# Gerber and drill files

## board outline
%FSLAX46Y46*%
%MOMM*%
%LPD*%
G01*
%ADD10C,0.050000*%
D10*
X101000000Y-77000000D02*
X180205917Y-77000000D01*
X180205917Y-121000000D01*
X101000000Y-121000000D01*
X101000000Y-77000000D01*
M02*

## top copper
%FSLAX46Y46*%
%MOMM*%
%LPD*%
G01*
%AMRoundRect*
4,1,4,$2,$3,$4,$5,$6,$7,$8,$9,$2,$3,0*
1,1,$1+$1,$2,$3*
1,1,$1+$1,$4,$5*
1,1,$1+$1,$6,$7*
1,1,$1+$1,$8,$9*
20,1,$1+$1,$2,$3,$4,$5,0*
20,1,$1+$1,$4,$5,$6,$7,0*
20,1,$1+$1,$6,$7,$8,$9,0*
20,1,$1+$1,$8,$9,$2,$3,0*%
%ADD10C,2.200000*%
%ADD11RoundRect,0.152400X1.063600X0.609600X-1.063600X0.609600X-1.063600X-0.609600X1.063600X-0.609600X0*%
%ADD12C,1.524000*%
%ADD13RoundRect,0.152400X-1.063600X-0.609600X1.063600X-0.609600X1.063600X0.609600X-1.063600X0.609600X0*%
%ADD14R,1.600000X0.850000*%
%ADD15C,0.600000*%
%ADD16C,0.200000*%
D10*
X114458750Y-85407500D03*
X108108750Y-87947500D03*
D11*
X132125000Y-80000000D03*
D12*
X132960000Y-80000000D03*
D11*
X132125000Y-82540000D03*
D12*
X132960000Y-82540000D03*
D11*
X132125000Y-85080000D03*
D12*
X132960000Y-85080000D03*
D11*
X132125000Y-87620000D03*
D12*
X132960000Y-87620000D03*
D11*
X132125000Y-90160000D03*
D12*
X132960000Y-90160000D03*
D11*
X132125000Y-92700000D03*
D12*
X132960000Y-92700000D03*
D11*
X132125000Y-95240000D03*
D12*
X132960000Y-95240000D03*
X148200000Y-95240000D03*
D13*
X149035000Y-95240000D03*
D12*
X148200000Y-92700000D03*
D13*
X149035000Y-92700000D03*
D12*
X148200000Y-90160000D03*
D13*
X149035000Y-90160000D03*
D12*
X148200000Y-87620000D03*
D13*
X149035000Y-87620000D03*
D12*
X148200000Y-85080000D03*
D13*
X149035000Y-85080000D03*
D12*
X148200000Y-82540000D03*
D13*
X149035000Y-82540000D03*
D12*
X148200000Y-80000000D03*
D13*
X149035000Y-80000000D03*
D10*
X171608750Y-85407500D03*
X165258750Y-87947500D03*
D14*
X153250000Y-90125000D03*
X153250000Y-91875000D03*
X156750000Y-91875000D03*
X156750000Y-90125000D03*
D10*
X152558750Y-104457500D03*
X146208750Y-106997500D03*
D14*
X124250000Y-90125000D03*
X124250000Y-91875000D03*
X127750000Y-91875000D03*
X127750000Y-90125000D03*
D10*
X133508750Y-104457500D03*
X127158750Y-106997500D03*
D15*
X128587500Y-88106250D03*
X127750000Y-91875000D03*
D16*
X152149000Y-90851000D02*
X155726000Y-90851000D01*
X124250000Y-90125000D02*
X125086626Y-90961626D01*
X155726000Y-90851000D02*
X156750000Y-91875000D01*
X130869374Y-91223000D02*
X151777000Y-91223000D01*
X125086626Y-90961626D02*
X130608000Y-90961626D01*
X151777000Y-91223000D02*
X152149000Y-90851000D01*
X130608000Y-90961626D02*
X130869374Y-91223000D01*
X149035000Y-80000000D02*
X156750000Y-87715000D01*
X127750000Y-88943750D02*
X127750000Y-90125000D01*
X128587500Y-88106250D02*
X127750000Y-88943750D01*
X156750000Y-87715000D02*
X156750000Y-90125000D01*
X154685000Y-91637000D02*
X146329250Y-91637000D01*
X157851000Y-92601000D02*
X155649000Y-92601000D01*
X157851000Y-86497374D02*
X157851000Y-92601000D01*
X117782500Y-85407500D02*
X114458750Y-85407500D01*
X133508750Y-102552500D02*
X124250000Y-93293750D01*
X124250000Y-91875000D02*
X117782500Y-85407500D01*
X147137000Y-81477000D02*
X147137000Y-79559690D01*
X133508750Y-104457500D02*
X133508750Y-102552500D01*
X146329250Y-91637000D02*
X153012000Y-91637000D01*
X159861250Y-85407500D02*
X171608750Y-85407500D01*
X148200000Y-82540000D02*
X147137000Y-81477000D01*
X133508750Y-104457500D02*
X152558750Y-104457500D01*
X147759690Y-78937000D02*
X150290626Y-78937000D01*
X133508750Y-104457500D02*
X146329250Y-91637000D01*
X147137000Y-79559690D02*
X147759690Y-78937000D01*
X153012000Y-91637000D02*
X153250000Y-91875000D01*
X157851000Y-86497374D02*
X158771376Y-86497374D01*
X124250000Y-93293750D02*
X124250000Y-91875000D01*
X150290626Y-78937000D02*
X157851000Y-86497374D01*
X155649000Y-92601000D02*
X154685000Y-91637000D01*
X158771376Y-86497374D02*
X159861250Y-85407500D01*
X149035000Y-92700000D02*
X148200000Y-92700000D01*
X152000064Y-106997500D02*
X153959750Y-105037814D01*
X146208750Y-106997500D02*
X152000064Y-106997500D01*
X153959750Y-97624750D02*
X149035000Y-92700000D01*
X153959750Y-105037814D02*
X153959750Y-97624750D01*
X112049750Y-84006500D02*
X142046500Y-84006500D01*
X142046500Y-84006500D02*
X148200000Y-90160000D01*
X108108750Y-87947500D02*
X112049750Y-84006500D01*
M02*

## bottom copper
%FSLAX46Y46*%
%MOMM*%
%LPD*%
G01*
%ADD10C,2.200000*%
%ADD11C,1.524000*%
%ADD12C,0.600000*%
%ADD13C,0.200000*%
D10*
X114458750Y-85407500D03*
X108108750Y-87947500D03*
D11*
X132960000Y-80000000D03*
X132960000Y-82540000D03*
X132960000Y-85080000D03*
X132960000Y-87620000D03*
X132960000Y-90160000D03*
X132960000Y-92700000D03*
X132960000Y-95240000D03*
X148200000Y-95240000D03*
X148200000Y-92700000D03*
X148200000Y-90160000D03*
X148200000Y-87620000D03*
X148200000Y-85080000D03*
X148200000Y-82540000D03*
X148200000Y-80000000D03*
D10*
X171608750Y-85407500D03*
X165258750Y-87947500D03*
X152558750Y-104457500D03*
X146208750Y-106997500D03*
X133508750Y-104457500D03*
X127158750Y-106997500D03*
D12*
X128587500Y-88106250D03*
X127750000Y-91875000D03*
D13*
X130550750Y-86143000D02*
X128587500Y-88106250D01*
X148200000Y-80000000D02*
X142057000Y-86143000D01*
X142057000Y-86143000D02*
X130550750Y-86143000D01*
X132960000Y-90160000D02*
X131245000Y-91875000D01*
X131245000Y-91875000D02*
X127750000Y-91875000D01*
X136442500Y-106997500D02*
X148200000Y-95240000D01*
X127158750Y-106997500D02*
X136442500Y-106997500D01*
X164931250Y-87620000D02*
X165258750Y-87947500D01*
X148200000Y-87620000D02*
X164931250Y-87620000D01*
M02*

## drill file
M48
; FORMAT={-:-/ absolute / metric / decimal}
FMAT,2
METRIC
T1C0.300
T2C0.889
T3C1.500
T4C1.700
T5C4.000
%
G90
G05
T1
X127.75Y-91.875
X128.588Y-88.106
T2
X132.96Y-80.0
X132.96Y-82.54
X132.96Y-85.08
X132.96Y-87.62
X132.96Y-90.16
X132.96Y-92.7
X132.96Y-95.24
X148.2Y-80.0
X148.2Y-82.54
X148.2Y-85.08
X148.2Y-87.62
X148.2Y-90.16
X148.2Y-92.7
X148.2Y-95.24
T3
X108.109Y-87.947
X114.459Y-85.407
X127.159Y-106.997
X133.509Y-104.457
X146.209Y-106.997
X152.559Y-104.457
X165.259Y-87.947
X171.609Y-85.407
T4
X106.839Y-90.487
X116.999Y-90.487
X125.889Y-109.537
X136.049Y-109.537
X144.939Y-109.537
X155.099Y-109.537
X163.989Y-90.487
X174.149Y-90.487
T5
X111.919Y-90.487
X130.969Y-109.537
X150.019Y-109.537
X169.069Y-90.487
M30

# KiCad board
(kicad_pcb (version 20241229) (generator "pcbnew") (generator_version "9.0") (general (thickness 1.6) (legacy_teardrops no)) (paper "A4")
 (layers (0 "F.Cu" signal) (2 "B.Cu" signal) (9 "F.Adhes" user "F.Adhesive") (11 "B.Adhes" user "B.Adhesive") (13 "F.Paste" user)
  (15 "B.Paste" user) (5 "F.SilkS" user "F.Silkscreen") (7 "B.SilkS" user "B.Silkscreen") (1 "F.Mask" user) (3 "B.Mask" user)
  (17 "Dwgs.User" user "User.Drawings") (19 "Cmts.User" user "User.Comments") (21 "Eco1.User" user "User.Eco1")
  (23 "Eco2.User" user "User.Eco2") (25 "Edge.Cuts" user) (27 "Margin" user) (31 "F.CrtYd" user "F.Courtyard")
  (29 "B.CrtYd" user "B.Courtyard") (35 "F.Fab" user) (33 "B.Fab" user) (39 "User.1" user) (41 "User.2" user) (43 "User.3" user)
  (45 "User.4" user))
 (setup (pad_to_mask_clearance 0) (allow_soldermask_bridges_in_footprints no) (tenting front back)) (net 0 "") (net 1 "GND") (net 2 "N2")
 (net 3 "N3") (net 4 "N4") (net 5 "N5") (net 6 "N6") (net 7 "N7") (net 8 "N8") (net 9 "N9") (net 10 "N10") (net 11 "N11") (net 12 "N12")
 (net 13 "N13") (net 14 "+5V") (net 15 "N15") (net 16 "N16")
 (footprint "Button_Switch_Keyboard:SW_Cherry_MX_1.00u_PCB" (layer "F.Cu") (at 114.45875 85.4075)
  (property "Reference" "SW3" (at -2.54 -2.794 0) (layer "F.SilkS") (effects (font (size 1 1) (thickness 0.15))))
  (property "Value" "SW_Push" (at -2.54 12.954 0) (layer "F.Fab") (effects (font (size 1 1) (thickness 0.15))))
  (pad "" np_thru_hole circle (at -7.62 5.08) (size 1.7 1.7) (drill 1.7) (layers "*.Cu" "*.Mask"))
  (pad "" np_thru_hole circle (at -2.54 5.08) (size 4 4) (drill 4) (layers "*.Cu" "*.Mask"))
  (pad "" np_thru_hole circle (at 2.54 5.08) (size 1.7 1.7) (drill 1.7) (layers "*.Cu" "*.Mask"))
  (pad "1" thru_hole circle (at 0 0) (size 2.2 2.2) (drill 1.5) (layers "*.Cu" "*.Mask") (remove_unused_layers no) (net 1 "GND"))
  (pad "2" thru_hole circle (at -6.35 2.54) (size 2.2 2.2) (drill 1.5) (layers "*.Cu" "*.Mask") (remove_unused_layers no) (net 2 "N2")))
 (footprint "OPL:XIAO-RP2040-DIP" (layer "F.Cu") (at 140.58 87.62)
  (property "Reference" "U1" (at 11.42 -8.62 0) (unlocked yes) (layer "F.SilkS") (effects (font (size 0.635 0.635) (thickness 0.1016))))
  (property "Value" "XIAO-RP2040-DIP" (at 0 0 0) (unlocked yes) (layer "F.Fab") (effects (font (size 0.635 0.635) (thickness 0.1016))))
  (pad "1" smd roundrect (at -8.455 -7.62 180) (size 2.432 1.524) (layers "F.Cu" "F.Mask") (roundrect_rratio 0.1) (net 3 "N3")
   (thermal_bridge_angle 45))
  (pad "1" thru_hole circle (at -7.62 -7.62 180) (size 1.524 1.524) (drill 0.889) (layers "*.Cu" "*.Mask") (remove_unused_layers no)
   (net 3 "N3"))
  (pad "2" smd roundrect (at -8.455 -5.08 180) (size 2.432 1.524) (layers "F.Cu" "F.Mask") (roundrect_rratio 0.1) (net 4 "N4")
   (thermal_bridge_angle 45))
  (pad "2" thru_hole circle (at -7.62 -5.08 180) (size 1.524 1.524) (drill 0.889) (layers "*.Cu" "*.Mask") (remove_unused_layers no)
   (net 4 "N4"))
  (pad "3" smd roundrect (at -8.455 -2.54 180) (size 2.432 1.524) (layers "F.Cu" "F.Mask") (roundrect_rratio 0.1) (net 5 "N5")
   (thermal_bridge_angle 45))
  (pad "3" thru_hole circle (at -7.62 -2.54 180) (size 1.524 1.524) (drill 0.889) (layers "*.Cu" "*.Mask") (remove_unused_layers no)
   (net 5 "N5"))
  (pad "4" smd roundrect (at -8.455 0 180) (size 2.432 1.524) (layers "F.Cu" "F.Mask") (roundrect_rratio 0.1) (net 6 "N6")
   (thermal_bridge_angle 45))
  (pad "4" thru_hole circle (at -7.62 0 180) (size 1.524 1.524) (drill 0.889) (layers "*.Cu" "*.Mask") (remove_unused_layers no)
   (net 6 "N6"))
  (pad "5" smd roundrect (at -8.455 2.54 180) (size 2.432 1.524) (layers "F.Cu" "F.Mask") (roundrect_rratio 0.1) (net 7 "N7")
   (thermal_bridge_angle 45))
  (pad "5" thru_hole circle (at -7.62 2.54 180) (size 1.524 1.524) (drill 0.889) (layers "*.Cu" "*.Mask") (remove_unused_layers no)
   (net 7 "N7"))
  (pad "6" smd roundrect (at -8.455 5.08 180) (size 2.432 1.524) (layers "F.Cu" "F.Mask") (roundrect_rratio 0.1) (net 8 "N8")
   (thermal_bridge_angle 45))
  (pad "6" thru_hole circle (at -7.62 5.08 180) (size 1.524 1.524) (drill 0.889) (layers "*.Cu" "*.Mask") (remove_unused_layers no)
   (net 8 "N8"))
  (pad "7" smd roundrect (at -8.455 7.62 180) (size 2.432 1.524) (layers "F.Cu" "F.Mask") (roundrect_rratio 0.1) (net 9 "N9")
   (thermal_bridge_angle 45))
  (pad "7" thru_hole circle (at -7.62 7.62 180) (size 1.524 1.524) (drill 0.889) (layers "*.Cu" "*.Mask") (remove_unused_layers no)
   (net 9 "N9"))
  (pad "8" thru_hole circle (at 7.62 7.62) (size 1.524 1.524) (drill 0.889) (layers "*.Cu" "*.Mask") (remove_unused_layers no)
   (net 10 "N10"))
  (pad "8" smd roundrect (at 8.455 7.62) (size 2.432 1.524) (layers "F.Cu" "F.Mask") (roundrect_rratio 0.1) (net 10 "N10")
   (thermal_bridge_angle 45))
  (pad "9" thru_hole circle (at 7.62 5.08) (size 1.524 1.524) (drill 0.889) (layers "*.Cu" "*.Mask") (remove_unused_layers no)
   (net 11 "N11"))
  (pad "9" smd roundrect (at 8.455 5.08) (size 2.432 1.524) (layers "F.Cu" "F.Mask") (roundrect_rratio 0.1) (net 11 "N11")
   (thermal_bridge_angle 45))
  (pad "10" thru_hole circle (at 7.62 2.54) (size 1.524 1.524) (drill 0.889) (layers "*.Cu" "*.Mask") (remove_unused_layers no) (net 2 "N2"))
  (pad "10" smd roundrect (at 8.455 2.54) (size 2.432 1.524) (layers "F.Cu" "F.Mask") (roundrect_rratio 0.1) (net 2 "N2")
   (thermal_bridge_angle 45))
  (pad "11" thru_hole circle (at 7.62 0) (size 1.524 1.524) (drill 0.889) (layers "*.Cu" "*.Mask") (remove_unused_layers no) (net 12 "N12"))
  (pad "11" smd roundrect (at 8.455 0) (size 2.432 1.524) (layers "F.Cu" "F.Mask") (roundrect_rratio 0.1) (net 12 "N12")
   (thermal_bridge_angle 45))
  (pad "12" thru_hole circle (at 7.62 -2.54) (size 1.524 1.524) (drill 0.889) (layers "*.Cu" "*.Mask") (remove_unused_layers no)
   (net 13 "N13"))
  (pad "12" smd roundrect (at 8.455 -2.54) (size 2.432 1.524) (layers "F.Cu" "F.Mask") (roundrect_rratio 0.1) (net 13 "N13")
   (thermal_bridge_angle 45))
  (pad "13" thru_hole circle (at 7.62 -5.08) (size 1.524 1.524) (drill 0.889) (layers "*.Cu" "*.Mask") (remove_unused_layers no)
   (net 1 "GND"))
  (pad "13" smd roundrect (at 8.455 -5.08) (size 2.432 1.524) (layers "F.Cu" "F.Mask") (roundrect_rratio 0.1) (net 1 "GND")
   (thermal_bridge_angle 45))
  (pad "14" thru_hole circle (at 7.62 -7.62) (size 1.524 1.524) (drill 0.889) (layers "*.Cu" "*.Mask") (remove_unused_layers no)
   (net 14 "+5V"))
  (pad "14" smd roundrect (at 8.455 -7.62) (size 2.432 1.524) (layers "F.Cu" "F.Mask") (roundrect_rratio 0.1) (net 14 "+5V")
   (thermal_bridge_angle 45)))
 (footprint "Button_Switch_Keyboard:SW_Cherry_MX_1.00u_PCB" (layer "F.Cu") (at 171.60875 85.4075)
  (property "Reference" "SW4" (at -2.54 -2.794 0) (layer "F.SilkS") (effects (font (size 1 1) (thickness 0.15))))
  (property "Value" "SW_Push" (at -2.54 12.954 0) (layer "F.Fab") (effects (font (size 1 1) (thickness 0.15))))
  (pad "" np_thru_hole circle (at -7.62 5.08) (size 1.7 1.7) (drill 1.7) (layers "*.Cu" "*.Mask"))
  (pad "" np_thru_hole circle (at -2.54 5.08) (size 4 4) (drill 4) (layers "*.Cu" "*.Mask"))
  (pad "" np_thru_hole circle (at 2.54 5.08) (size 1.7 1.7) (drill 1.7) (layers "*.Cu" "*.Mask"))
  (pad "1" thru_hole circle (at 0 0) (size 2.2 2.2) (drill 1.5) (layers "*.Cu" "*.Mask") (remove_unused_layers no) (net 1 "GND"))
  (pad "2" thru_hole circle (at -6.35 2.54) (size 2.2 2.2) (drill 1.5) (layers "*.Cu" "*.Mask") (remove_unused_layers no) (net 12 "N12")))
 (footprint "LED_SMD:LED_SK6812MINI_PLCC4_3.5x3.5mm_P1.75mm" (layer "F.Cu") (at 155 91)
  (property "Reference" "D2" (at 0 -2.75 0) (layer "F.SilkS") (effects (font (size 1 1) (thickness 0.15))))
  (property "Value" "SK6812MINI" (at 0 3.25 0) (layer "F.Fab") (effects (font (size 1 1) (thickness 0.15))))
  (pad "1" smd rect (at -1.75 -0.875) (size 1.6 0.85) (layers "F.Cu" "F.Mask" "F.Paste") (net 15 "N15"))
  (pad "2" smd rect (at -1.75 0.875) (size 1.6 0.85) (layers "F.Cu" "F.Mask" "F.Paste") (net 1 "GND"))
  (pad "3" smd rect (at 1.75 0.875) (size 1.6 0.85) (layers "F.Cu" "F.Mask" "F.Paste") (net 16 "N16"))
  (pad "4" smd rect (at 1.75 -0.875) (size 1.6 0.85) (layers "F.Cu" "F.Mask" "F.Paste") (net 14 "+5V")))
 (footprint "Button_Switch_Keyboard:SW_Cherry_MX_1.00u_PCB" (layer "F.Cu") (at 152.55875 104.4575)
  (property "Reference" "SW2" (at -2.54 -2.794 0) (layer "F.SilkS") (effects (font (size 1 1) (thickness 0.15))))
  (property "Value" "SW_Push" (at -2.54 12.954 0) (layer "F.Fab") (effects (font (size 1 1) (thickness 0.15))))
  (pad "" np_thru_hole circle (at -7.62 5.08) (size 1.7 1.7) (drill 1.7) (layers "*.Cu" "*.Mask"))
  (pad "" np_thru_hole circle (at -2.54 5.08) (size 4 4) (drill 4) (layers "*.Cu" "*.Mask"))
  (pad "" np_thru_hole circle (at 2.54 5.08) (size 1.7 1.7) (drill 1.7) (layers "*.Cu" "*.Mask"))
  (pad "1" thru_hole circle (at 0 0) (size 2.2 2.2) (drill 1.5) (layers "*.Cu" "*.Mask") (remove_unused_layers no) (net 1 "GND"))
  (pad "2" thru_hole circle (at -6.35 2.54) (size 2.2 2.2) (drill 1.5) (layers "*.Cu" "*.Mask") (remove_unused_layers no) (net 11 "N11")))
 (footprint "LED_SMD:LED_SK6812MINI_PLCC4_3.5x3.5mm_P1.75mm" (layer "F.Cu") (at 126 91)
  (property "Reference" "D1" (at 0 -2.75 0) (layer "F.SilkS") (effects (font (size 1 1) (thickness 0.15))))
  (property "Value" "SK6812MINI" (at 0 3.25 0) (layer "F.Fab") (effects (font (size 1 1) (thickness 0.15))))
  (pad "1" smd rect (at -1.75 -0.875) (size 1.6 0.85) (layers "F.Cu" "F.Mask" "F.Paste") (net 16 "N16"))
  (pad "2" smd rect (at -1.75 0.875) (size 1.6 0.85) (layers "F.Cu" "F.Mask" "F.Paste") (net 1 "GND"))
  (pad "3" smd rect (at 1.75 0.875) (size 1.6 0.85) (layers "F.Cu" "F.Mask" "F.Paste") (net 7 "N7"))
  (pad "4" smd rect (at 1.75 -0.875) (size 1.6 0.85) (layers "F.Cu" "F.Mask" "F.Paste") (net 14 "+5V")))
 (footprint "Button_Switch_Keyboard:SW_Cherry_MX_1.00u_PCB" (layer "F.Cu") (at 133.50875 104.4575)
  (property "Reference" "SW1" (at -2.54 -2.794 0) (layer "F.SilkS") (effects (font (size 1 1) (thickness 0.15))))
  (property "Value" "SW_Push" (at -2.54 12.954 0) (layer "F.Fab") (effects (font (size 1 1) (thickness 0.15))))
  (pad "" np_thru_hole circle (at -7.62 5.08) (size 1.7 1.7) (drill 1.7) (layers "*.Cu" "*.Mask"))
  (pad "" np_thru_hole circle (at -2.54 5.08) (size 4 4) (drill 4) (layers "*.Cu" "*.Mask"))
  (pad "" np_thru_hole circle (at 2.54 5.08) (size 1.7 1.7) (drill 1.7) (layers "*.Cu" "*.Mask"))
  (pad "1" thru_hole circle (at 0 0) (size 2.2 2.2) (drill 1.5) (layers "*.Cu" "*.Mask") (remove_unused_layers no) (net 1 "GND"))
  (pad "2" thru_hole circle (at -6.35 2.54) (size 2.2 2.2) (drill 1.5) (layers "*.Cu" "*.Mask") (remove_unused_layers no) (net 10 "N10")))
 (gr_rect (start 101 77) (end 180.205917 121) (stroke (width 0.05) (type default)) (fill no) (layer "Edge.Cuts"))
 (segment (start 152.149 90.851) (end 155.726 90.851) (width 0.2) (layer "F.Cu") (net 16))
 (segment (start 124.25 90.125) (end 125.086626 90.961626) (width 0.2) (layer "F.Cu") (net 16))
 (segment (start 155.726 90.851) (end 156.75 91.875) (width 0.2) (layer "F.Cu") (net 16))
 (segment (start 130.869374 91.223) (end 151.777 91.223) (width 0.2) (layer "F.Cu") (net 16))
 (segment (start 125.086626 90.961626) (end 130.608 90.961626) (width 0.2) (layer "F.Cu") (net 16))
 (segment (start 151.777 91.223) (end 152.149 90.851) (width 0.2) (layer "F.Cu") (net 16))
 (segment (start 130.608 90.961626) (end 130.869374 91.223) (width 0.2) (layer "F.Cu") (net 16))
 (segment (start 149.035 80) (end 156.75 87.715) (width 0.2) (layer "F.Cu") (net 14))
 (segment (start 127.75 88.94375) (end 127.75 90.125) (width 0.2) (layer "F.Cu") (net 14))
 (segment (start 128.5875 88.10625) (end 127.75 88.94375) (width 0.2) (layer "F.Cu") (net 14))
 (segment (start 156.75 87.715) (end 156.75 90.125) (width 0.2) (layer "F.Cu") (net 14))
 (via (at 128.5875 88.10625) (size 0.6) (drill 0.3) (layers "F.Cu" "B.Cu") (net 14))
 (segment (start 130.55075 86.143) (end 128.5875 88.10625) (width 0.2) (layer "B.Cu") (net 14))
 (segment (start 148.2 80) (end 142.057 86.143) (width 0.2) (layer "B.Cu") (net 14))
 (segment (start 142.057 86.143) (end 130.55075 86.143) (width 0.2) (layer "B.Cu") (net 14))
 (via (at 127.75 91.875) (size 0.6) (drill 0.3) (layers "F.Cu" "B.Cu") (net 7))
 (segment (start 132.96 90.16) (end 131.245 91.875) (width 0.2) (layer "B.Cu") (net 7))
 (segment (start 131.245 91.875) (end 127.75 91.875) (width 0.2) (layer "B.Cu") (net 7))
 (segment (start 154.685 91.637) (end 146.32925 91.637) (width 0.2) (layer "F.Cu") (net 1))
 (segment (start 157.851 92.601) (end 155.649 92.601) (width 0.2) (layer "F.Cu") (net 1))
 (segment (start 157.851 86.497374) (end 157.851 92.601) (width 0.2) (layer "F.Cu") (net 1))
 (segment (start 117.7825 85.4075) (end 114.45875 85.4075) (width 0.2) (layer "F.Cu") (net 1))
 (segment (start 133.50875 102.5525) (end 124.25 93.29375) (width 0.2) (layer "F.Cu") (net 1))
 (segment (start 124.25 91.875) (end 117.7825 85.4075) (width 0.2) (layer "F.Cu") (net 1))
 (segment (start 147.137 81.477) (end 147.137 79.55969) (width 0.2) (layer "F.Cu") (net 1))
 (segment (start 133.50875 104.4575) (end 133.50875 102.5525) (width 0.2) (layer "F.Cu") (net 1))
 (segment (start 146.32925 91.637) (end 153.012 91.637) (width 0.2) (layer "F.Cu") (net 1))
 (segment (start 159.86125 85.4075) (end 171.60875 85.4075) (width 0.2) (layer "F.Cu") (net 1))
 (segment (start 148.2 82.54) (end 147.137 81.477) (width 0.2) (layer "F.Cu") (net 1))
 (segment (start 133.50875 104.4575) (end 152.55875 104.4575) (width 0.2) (layer "F.Cu") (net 1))
 (segment (start 147.75969 78.937) (end 150.290626 78.937) (width 0.2) (layer "F.Cu") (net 1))
 (segment (start 133.50875 104.4575) (end 146.32925 91.637) (width 0.2) (layer "F.Cu") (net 1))
 (segment (start 147.137 79.55969) (end 147.75969 78.937) (width 0.2) (layer "F.Cu") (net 1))
 (segment (start 153.012 91.637) (end 153.25 91.875) (width 0.2) (layer "F.Cu") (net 1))
 (segment (start 157.851 86.497374) (end 158.771376 86.497374) (width 0.2) (layer "F.Cu") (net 1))
 (segment (start 124.25 93.29375) (end 124.25 91.875) (width 0.2) (layer "F.Cu") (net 1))
 (segment (start 150.290626 78.937) (end 157.851 86.497374) (width 0.2) (layer "F.Cu") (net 1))
 (segment (start 155.649 92.601) (end 154.685 91.637) (width 0.2) (layer "F.Cu") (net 1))
 (segment (start 158.771376 86.497374) (end 159.86125 85.4075) (width 0.2) (layer "F.Cu") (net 1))
 (segment (start 136.4425 106.9975) (end 148.2 95.24) (width 0.2) (layer "B.Cu") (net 10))
 (segment (start 127.15875 106.9975) (end 136.4425 106.9975) (width 0.2) (layer "B.Cu") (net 10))
 (segment (start 149.035 92.7) (end 148.2 92.7) (width 0.2) (layer "F.Cu") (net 11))
 (segment (start 152.000064 106.9975) (end 153.95975 105.037814) (width 0.2) (layer "F.Cu") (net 11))
 (segment (start 146.20875 106.9975) (end 152.000064 106.9975) (width 0.2) (layer "F.Cu") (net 11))
 (segment (start 153.95975 97.62475) (end 149.035 92.7) (width 0.2) (layer "F.Cu") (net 11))
 (segment (start 153.95975 105.037814) (end 153.95975 97.62475) (width 0.2) (layer "F.Cu") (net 11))
 (segment (start 112.04975 84.0065) (end 142.0465 84.0065) (width 0.2) (layer "F.Cu") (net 2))
 (segment (start 142.0465 84.0065) (end 148.2 90.16) (width 0.2) (layer "F.Cu") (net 2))
 (segment (start 108.10875 87.9475) (end 112.04975 84.0065) (width 0.2) (layer "F.Cu") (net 2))
 (segment (start 164.93125 87.62) (end 165.25875 87.9475) (width 0.2) (layer "B.Cu") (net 12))
 (segment (start 148.2 87.62) (end 164.93125 87.62) (width 0.2) (layer "B.Cu") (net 12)))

